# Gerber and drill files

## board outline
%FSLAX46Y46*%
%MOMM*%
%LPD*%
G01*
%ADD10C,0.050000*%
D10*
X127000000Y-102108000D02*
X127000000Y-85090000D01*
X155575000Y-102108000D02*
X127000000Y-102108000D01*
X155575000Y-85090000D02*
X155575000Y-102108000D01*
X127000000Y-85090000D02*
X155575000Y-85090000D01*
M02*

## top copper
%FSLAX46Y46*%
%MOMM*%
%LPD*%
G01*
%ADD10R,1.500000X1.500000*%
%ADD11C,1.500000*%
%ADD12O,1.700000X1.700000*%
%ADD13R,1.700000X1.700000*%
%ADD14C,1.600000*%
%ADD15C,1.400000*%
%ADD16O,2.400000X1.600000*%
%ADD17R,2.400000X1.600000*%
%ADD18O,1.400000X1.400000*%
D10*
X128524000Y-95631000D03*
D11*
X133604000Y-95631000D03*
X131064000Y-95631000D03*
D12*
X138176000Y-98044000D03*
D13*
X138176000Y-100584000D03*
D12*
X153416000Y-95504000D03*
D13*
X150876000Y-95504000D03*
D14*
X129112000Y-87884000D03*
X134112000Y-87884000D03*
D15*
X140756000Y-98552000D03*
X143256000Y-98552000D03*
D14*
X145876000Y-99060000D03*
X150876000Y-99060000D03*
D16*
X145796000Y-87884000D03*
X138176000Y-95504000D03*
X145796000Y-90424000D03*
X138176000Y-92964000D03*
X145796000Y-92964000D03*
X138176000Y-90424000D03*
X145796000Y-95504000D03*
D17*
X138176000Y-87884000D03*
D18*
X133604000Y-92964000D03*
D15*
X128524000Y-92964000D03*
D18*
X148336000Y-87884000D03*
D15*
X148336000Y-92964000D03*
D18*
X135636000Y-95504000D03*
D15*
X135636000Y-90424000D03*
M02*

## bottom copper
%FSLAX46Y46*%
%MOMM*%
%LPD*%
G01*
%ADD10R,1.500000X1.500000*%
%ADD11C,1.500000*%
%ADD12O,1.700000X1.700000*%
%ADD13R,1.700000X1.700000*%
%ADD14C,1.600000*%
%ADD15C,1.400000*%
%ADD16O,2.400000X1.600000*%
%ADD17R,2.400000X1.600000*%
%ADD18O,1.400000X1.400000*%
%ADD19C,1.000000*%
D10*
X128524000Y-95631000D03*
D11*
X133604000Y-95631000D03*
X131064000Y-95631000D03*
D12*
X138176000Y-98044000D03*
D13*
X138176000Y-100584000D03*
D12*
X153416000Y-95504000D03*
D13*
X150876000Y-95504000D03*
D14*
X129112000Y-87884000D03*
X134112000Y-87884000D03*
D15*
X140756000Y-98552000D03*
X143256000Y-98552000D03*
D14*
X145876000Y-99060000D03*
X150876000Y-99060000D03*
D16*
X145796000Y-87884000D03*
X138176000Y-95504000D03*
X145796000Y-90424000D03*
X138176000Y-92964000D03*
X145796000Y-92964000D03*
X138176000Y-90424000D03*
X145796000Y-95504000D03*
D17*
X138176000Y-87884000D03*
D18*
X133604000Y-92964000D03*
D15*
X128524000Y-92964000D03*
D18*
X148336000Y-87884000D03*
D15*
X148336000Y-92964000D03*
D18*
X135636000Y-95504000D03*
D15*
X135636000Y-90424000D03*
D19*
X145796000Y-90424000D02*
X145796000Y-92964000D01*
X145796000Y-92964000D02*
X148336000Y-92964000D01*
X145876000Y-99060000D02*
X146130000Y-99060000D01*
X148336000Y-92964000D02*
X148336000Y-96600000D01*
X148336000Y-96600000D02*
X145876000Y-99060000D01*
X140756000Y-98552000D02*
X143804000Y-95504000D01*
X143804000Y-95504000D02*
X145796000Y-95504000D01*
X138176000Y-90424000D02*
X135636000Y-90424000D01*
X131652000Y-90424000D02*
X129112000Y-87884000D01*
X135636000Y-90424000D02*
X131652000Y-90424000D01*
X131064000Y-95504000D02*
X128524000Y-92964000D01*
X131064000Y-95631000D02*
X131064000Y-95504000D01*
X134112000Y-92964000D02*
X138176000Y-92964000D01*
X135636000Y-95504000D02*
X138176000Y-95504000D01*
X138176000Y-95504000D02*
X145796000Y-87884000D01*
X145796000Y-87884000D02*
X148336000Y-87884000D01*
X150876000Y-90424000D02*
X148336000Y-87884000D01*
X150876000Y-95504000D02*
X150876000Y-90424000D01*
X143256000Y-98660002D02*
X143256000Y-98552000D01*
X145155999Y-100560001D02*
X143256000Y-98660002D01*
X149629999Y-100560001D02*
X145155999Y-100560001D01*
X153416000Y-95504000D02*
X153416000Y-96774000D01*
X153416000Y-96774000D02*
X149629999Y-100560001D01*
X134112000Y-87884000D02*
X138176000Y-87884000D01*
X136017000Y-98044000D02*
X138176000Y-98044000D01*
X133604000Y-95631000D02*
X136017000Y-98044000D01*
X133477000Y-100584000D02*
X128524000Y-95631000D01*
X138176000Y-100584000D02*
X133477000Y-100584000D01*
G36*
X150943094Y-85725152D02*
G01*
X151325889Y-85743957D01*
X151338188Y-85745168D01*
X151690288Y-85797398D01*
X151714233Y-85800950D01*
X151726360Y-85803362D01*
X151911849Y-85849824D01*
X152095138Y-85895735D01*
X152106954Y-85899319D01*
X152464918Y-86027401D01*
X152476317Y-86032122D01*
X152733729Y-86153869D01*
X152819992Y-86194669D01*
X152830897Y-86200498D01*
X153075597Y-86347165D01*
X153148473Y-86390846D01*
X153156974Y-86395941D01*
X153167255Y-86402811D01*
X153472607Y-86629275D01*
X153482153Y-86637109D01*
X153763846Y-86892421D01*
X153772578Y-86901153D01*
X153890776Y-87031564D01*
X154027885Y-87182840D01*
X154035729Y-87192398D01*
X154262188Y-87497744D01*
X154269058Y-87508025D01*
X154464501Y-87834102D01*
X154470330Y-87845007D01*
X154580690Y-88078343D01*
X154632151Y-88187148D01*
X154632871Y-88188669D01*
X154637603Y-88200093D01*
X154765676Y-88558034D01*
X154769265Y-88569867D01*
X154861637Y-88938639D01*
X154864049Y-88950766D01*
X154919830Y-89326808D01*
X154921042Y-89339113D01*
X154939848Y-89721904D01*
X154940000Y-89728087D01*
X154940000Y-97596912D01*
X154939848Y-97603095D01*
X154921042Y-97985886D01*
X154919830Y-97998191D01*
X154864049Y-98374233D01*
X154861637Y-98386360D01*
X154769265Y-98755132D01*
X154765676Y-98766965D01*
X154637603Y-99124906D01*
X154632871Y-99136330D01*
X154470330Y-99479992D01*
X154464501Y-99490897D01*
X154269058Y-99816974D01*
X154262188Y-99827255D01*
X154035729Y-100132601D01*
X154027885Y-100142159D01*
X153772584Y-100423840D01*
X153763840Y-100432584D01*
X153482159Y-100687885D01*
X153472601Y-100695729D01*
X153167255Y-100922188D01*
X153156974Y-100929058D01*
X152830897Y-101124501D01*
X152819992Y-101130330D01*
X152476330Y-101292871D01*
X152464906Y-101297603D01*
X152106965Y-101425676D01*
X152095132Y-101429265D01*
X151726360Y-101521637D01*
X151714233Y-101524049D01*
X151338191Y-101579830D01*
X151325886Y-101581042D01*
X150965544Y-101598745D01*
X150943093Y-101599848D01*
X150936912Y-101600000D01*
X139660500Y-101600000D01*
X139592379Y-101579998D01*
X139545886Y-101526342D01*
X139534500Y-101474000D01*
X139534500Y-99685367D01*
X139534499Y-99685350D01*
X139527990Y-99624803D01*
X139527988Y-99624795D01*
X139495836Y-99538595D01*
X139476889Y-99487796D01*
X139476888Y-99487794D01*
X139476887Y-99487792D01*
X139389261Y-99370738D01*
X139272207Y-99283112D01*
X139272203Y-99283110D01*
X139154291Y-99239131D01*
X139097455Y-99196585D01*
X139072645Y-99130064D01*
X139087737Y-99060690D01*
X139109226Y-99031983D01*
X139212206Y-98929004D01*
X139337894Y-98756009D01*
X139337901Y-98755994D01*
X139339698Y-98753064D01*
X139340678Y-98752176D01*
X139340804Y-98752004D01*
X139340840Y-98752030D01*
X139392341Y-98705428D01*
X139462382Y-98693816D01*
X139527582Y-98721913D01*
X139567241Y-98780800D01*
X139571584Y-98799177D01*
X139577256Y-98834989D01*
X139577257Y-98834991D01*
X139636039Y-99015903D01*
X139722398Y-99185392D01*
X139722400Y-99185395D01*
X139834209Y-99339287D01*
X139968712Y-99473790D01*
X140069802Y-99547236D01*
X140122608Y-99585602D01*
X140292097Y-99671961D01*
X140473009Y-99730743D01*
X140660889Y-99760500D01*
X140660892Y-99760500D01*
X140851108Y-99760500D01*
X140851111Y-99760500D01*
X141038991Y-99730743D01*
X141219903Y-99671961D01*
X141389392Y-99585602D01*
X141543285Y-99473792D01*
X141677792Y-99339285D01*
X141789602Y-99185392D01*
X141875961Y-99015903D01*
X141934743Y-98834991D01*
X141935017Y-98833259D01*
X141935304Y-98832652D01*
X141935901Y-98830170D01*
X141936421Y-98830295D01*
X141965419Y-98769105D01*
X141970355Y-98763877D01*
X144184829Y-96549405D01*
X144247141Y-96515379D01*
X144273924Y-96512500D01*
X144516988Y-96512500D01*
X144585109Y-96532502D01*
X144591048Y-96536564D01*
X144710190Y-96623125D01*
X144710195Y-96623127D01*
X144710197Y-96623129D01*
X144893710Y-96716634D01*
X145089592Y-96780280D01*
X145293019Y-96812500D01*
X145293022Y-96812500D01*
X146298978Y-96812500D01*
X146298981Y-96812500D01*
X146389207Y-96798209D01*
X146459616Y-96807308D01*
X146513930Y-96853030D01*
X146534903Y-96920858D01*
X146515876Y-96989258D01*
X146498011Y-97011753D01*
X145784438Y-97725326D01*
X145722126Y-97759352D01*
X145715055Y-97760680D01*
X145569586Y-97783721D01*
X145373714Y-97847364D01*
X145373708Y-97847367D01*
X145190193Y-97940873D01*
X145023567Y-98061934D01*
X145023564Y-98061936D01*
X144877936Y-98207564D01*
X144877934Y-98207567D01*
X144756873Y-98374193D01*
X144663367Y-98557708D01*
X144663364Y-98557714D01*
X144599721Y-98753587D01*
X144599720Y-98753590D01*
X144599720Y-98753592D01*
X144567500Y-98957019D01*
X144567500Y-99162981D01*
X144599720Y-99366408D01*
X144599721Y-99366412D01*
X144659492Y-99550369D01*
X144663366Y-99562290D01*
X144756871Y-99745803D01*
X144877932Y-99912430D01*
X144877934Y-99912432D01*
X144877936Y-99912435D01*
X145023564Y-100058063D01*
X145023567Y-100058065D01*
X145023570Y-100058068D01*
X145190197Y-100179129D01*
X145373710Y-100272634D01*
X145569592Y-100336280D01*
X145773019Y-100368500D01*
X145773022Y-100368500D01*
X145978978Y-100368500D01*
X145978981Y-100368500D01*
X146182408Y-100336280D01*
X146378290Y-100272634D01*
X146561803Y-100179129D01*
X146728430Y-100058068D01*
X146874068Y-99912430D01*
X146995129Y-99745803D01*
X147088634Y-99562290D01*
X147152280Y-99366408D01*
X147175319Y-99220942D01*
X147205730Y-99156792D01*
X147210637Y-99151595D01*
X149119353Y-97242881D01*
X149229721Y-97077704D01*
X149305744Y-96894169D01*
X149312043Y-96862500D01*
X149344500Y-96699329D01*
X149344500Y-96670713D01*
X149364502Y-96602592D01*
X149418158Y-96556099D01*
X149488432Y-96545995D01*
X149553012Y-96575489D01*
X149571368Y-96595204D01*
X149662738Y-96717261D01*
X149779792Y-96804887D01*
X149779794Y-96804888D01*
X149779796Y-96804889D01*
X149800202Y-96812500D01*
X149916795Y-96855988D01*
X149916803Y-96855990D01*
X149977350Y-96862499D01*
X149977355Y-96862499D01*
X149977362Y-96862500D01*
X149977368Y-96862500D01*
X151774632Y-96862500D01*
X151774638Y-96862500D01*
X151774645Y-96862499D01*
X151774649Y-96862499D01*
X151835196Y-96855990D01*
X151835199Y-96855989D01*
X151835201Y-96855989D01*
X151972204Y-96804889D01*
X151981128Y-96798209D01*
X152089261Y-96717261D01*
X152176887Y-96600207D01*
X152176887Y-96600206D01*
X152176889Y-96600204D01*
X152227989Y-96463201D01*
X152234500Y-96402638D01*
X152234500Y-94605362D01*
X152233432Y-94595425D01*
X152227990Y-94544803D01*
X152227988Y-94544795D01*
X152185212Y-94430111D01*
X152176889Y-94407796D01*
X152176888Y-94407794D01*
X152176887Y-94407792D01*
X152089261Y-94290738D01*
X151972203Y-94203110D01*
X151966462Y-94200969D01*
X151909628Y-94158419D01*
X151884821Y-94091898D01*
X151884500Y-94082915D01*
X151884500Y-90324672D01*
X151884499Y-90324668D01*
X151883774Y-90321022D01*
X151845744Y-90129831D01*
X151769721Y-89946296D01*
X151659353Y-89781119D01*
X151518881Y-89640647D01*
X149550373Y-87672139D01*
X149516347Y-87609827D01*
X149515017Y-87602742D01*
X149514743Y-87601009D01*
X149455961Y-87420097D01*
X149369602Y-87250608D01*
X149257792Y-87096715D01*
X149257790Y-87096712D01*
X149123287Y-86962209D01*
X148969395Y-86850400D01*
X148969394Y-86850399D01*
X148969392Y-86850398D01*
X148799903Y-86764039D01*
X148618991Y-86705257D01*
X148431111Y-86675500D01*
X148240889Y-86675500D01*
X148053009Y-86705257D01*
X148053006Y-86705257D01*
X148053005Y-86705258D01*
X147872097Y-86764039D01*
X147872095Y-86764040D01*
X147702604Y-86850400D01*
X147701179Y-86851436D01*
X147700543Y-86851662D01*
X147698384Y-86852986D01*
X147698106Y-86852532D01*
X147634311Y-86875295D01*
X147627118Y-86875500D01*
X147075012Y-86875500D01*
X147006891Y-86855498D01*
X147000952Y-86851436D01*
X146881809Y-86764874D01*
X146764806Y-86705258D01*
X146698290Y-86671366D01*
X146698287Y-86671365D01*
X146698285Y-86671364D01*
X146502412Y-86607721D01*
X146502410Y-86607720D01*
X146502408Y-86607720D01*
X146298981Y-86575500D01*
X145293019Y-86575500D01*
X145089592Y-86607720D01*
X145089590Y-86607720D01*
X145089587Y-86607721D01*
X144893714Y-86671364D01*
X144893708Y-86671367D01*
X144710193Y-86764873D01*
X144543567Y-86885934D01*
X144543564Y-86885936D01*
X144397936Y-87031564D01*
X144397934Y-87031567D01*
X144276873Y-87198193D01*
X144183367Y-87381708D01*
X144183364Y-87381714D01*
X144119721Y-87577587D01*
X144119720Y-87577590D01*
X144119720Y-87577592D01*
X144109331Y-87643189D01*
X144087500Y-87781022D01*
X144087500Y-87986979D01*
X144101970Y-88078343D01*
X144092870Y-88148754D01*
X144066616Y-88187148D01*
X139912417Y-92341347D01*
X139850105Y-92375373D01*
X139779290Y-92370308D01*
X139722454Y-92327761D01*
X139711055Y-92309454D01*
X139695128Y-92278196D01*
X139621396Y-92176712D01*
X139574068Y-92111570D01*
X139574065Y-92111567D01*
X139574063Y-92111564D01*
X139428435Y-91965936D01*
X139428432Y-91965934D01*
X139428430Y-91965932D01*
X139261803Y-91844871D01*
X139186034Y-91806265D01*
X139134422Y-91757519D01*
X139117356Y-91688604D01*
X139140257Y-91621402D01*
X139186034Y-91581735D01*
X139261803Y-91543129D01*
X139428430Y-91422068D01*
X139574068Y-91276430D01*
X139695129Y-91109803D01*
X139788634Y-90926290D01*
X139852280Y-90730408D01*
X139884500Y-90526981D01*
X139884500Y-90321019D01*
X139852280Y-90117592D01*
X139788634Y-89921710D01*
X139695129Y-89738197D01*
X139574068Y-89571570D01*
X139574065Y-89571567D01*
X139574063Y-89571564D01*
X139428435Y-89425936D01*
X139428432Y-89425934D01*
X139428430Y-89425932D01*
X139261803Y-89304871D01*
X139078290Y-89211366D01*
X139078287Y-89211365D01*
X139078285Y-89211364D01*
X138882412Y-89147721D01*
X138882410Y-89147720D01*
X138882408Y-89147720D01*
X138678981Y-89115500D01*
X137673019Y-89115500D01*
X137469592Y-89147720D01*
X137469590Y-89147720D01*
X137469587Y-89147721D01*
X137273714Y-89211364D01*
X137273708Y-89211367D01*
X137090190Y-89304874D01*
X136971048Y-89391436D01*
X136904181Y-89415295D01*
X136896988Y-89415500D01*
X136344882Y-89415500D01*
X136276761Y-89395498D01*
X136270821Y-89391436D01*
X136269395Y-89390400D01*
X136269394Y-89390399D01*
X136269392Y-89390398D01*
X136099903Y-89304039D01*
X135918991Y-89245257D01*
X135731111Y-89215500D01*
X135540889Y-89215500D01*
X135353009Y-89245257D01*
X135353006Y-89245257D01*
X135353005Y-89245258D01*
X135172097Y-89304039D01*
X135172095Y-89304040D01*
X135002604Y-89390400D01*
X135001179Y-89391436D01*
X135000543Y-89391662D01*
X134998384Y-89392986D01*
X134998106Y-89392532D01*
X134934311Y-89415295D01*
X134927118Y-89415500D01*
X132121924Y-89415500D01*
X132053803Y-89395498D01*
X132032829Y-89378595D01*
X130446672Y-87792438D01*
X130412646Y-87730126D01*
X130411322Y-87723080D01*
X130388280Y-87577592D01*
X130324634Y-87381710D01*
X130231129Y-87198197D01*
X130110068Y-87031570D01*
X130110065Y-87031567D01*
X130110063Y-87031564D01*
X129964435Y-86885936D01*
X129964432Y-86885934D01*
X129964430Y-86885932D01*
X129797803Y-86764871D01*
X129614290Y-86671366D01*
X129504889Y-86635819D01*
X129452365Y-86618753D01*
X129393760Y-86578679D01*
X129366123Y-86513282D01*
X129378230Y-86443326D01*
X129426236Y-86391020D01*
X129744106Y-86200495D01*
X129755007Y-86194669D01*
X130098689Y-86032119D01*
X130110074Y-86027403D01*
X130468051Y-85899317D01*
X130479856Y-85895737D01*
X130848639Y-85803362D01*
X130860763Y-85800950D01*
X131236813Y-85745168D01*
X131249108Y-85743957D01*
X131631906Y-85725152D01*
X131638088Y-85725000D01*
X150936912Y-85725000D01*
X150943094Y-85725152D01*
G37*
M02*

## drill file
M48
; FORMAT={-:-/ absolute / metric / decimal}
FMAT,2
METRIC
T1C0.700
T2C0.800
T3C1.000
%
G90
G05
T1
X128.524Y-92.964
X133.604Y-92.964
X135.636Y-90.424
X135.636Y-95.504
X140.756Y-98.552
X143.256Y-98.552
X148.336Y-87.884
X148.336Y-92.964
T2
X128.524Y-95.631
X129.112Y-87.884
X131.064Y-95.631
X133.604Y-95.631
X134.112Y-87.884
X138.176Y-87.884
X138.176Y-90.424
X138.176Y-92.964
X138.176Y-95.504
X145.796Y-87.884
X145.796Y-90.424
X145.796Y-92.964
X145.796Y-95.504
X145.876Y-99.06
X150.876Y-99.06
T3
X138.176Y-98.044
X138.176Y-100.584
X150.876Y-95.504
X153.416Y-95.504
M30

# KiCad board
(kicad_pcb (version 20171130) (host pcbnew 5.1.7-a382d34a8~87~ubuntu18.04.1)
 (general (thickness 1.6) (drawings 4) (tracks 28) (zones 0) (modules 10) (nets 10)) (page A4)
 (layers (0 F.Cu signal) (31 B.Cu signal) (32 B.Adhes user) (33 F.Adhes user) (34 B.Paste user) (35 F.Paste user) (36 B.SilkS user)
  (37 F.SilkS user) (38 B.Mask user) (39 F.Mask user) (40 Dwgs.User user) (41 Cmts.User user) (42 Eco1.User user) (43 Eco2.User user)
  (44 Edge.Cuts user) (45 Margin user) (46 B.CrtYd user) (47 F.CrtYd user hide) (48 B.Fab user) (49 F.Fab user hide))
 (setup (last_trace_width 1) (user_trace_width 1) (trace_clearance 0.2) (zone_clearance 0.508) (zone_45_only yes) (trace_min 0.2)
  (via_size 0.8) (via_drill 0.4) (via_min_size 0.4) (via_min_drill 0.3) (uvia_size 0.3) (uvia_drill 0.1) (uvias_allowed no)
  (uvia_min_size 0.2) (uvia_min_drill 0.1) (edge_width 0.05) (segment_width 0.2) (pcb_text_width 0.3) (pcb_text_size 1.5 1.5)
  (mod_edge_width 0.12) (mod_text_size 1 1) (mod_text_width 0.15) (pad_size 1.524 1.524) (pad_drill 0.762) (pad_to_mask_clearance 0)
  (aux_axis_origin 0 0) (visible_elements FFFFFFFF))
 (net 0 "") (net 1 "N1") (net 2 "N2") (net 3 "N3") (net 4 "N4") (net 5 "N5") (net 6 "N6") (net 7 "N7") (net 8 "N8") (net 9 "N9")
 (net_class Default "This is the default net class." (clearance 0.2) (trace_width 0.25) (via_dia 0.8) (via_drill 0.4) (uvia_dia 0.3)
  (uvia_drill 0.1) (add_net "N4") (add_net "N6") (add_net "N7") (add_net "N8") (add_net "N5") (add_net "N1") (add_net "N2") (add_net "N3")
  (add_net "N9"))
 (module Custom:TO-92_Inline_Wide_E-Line (layer F.Cu) (at 128.524 95.631)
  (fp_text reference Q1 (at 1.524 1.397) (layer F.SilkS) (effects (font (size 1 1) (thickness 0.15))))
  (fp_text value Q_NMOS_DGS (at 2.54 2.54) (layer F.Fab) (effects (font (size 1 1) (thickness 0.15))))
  (pad 1 thru_hole rect (at 0 0 90) (size 1.5 1.5) (drill 0.8) (layers *.Cu *.Mask) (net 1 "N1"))
  (pad 3 thru_hole circle (at 5.08 0 90) (size 1.5 1.5) (drill 0.8) (layers *.Cu *.Mask) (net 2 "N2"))
  (pad 2 thru_hole circle (at 2.54 0 90) (size 1.5 1.5) (drill 0.8) (layers *.Cu *.Mask) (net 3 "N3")))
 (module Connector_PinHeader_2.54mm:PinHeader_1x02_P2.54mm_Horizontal (layer F.Cu) (at 138.176 100.584 180)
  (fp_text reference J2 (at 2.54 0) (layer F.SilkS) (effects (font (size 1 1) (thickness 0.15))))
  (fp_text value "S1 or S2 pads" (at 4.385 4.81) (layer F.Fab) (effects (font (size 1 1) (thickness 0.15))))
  (pad 2 thru_hole oval (at 0 2.54 180) (size 1.7 1.7) (drill 1) (layers *.Cu *.Mask) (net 2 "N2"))
  (pad 1 thru_hole rect (at 0 0 180) (size 1.7 1.7) (drill 1) (layers *.Cu *.Mask) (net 1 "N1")))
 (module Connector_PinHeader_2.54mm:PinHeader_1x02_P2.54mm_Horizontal (layer F.Cu) (at 150.876 95.504 90)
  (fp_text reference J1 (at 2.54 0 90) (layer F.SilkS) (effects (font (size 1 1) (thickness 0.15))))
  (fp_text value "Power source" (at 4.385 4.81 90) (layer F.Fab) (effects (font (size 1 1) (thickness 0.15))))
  (pad 2 thru_hole oval (at 0 2.54 90) (size 1.7 1.7) (drill 1) (layers *.Cu *.Mask) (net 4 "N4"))
  (pad 1 thru_hole rect (at 0 0 90) (size 1.7 1.7) (drill 1) (layers *.Cu *.Mask) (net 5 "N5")))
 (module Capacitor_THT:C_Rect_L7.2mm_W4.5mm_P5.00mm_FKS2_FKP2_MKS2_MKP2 (layer F.Cu) (at 134.112 87.884 180)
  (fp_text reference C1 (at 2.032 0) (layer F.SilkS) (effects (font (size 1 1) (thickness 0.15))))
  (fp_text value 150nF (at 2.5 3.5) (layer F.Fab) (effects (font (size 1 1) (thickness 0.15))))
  (pad 2 thru_hole circle (at 5 0 180) (size 1.6 1.6) (drill 0.8) (layers *.Cu *.Mask) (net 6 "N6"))
  (pad 1 thru_hole circle (at 0 0 180) (size 1.6 1.6) (drill 0.8) (layers *.Cu *.Mask) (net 4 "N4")))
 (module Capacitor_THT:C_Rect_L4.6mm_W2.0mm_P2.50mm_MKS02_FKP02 (layer F.Cu) (at 143.256 98.552 180)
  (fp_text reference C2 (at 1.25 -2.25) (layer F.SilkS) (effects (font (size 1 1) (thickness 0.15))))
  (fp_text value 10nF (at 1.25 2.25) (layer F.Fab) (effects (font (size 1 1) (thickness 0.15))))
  (pad 2 thru_hole circle (at 2.5 0 180) (size 1.4 1.4) (drill 0.7) (layers *.Cu *.Mask) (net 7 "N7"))
  (pad 1 thru_hole circle (at 0 0 180) (size 1.4 1.4) (drill 0.7) (layers *.Cu *.Mask) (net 4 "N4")))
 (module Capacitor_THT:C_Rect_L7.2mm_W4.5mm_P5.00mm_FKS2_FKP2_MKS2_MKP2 (layer F.Cu) (at 150.876 99.06 180)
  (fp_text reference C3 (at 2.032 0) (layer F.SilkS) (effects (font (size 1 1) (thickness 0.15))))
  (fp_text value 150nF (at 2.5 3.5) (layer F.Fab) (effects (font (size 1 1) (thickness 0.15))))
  (pad 2 thru_hole circle (at 5 0 180) (size 1.6 1.6) (drill 0.8) (layers *.Cu *.Mask) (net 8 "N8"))
  (pad 1 thru_hole circle (at 0 0 180) (size 1.6 1.6) (drill 0.8) (layers *.Cu *.Mask) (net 4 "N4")))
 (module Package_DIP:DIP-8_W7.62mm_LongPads (layer F.Cu) (at 138.176 87.884)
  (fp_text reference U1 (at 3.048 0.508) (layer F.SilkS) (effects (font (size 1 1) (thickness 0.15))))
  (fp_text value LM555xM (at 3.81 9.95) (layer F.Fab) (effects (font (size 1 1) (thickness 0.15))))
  (pad 8 thru_hole oval (at 7.62 0) (size 2.4 1.6) (drill 0.8) (layers *.Cu *.Mask) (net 5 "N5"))
  (pad 4 thru_hole oval (at 0 7.62) (size 2.4 1.6) (drill 0.8) (layers *.Cu *.Mask) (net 5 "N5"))
  (pad 7 thru_hole oval (at 7.62 2.54) (size 2.4 1.6) (drill 0.8) (layers *.Cu *.Mask) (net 8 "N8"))
  (pad 3 thru_hole oval (at 0 5.08) (size 2.4 1.6) (drill 0.8) (layers *.Cu *.Mask) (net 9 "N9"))
  (pad 6 thru_hole oval (at 7.62 5.08) (size 2.4 1.6) (drill 0.8) (layers *.Cu *.Mask) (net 8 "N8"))
  (pad 2 thru_hole oval (at 0 2.54) (size 2.4 1.6) (drill 0.8) (layers *.Cu *.Mask) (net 6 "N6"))
  (pad 5 thru_hole oval (at 7.62 7.62) (size 2.4 1.6) (drill 0.8) (layers *.Cu *.Mask) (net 7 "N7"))
  (pad 1 thru_hole rect (at 0 0) (size 2.4 1.6) (drill 0.8) (layers *.Cu *.Mask) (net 4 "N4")))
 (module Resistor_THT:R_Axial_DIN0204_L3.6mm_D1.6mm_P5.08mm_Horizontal (layer F.Cu) (at 128.524 92.964)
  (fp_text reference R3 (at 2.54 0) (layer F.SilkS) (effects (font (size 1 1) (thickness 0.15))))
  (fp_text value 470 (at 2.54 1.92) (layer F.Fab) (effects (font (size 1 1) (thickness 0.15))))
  (pad 2 thru_hole oval (at 5.08 0) (size 1.4 1.4) (drill 0.7) (layers *.Cu *.Mask) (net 9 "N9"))
  (pad 1 thru_hole circle (at 0 0) (size 1.4 1.4) (drill 0.7) (layers *.Cu *.Mask) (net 3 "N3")))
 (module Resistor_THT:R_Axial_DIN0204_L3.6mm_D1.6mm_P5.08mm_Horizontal (layer F.Cu) (at 148.336 92.964 90)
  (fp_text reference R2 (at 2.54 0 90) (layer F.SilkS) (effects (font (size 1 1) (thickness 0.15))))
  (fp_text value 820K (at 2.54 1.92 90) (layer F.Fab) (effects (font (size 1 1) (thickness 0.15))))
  (pad 2 thru_hole oval (at 5.08 0 90) (size 1.4 1.4) (drill 0.7) (layers *.Cu *.Mask) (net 5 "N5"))
  (pad 1 thru_hole circle (at 0 0 90) (size 1.4 1.4) (drill 0.7) (layers *.Cu *.Mask) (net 8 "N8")))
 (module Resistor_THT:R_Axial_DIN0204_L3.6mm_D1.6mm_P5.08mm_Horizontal (layer F.Cu) (at 135.636 90.424 270)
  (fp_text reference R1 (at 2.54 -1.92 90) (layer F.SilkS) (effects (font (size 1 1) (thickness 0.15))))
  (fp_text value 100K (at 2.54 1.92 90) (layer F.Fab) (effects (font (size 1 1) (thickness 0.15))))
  (pad 2 thru_hole oval (at 5.08 0 270) (size 1.4 1.4) (drill 0.7) (layers *.Cu *.Mask) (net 5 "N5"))
  (pad 1 thru_hole circle (at 0 0 270) (size 1.4 1.4) (drill 0.7) (layers *.Cu *.Mask) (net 6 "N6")))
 (gr_line (start 127 102.108) (end 127 85.09) (layer Edge.Cuts) (width 0.05))
 (gr_line (start 155.575 102.108) (end 127 102.108) (layer Edge.Cuts) (width 0.05))
 (gr_line (start 155.575 85.09) (end 155.575 102.108) (layer Edge.Cuts) (width 0.05))
 (gr_line (start 127 85.09) (end 155.575 85.09) (layer Edge.Cuts) (width 0.05))
 (segment (start 145.796 90.424) (end 145.796 92.964) (width 1) (layer B.Cu) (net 8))
 (segment (start 145.796 92.964) (end 148.336 92.964) (width 1) (layer B.Cu) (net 8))
 (segment (start 145.876 99.06) (end 146.13 99.06) (width 1) (layer B.Cu) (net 8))
 (segment (start 148.336 92.964) (end 148.336 96.6) (width 1) (layer B.Cu) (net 8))
 (segment (start 148.336 96.6) (end 145.876 99.06) (width 1) (layer B.Cu) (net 8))
 (segment (start 140.756 98.552) (end 143.804 95.504) (width 1) (layer B.Cu) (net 7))
 (segment (start 143.804 95.504) (end 145.796 95.504) (width 1) (layer B.Cu) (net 7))
 (segment (start 138.176 90.424) (end 135.636 90.424) (width 1) (layer B.Cu) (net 6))
 (segment (start 131.652 90.424) (end 129.112 87.884) (width 1) (layer B.Cu) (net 6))
 (segment (start 135.636 90.424) (end 131.652 90.424) (width 1) (layer B.Cu) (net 6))
 (segment (start 131.064 95.504) (end 128.524 92.964) (width 1) (layer B.Cu) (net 3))
 (segment (start 131.064 95.631) (end 131.064 95.504) (width 1) (layer B.Cu) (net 3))
 (segment (start 134.112 92.964) (end 138.176 92.964) (width 1) (layer B.Cu) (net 9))
 (segment (start 135.636 95.504) (end 138.176 95.504) (width 1) (layer B.Cu) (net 5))
 (segment (start 138.176 95.504) (end 145.796 87.884) (width 1) (layer B.Cu) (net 5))
 (segment (start 145.796 87.884) (end 148.336 87.884) (width 1) (layer B.Cu) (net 5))
 (segment (start 150.876 90.424) (end 148.336 87.884) (width 1) (layer B.Cu) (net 5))
 (segment (start 150.876 95.504) (end 150.876 90.424) (width 1) (layer B.Cu) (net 5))
 (segment (start 143.256 98.660002) (end 143.256 98.552) (width 1) (layer B.Cu) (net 4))
 (segment (start 145.155999 100.560001) (end 143.256 98.660002) (width 1) (layer B.Cu) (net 4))
 (segment (start 149.629999 100.560001) (end 145.155999 100.560001) (width 1) (layer B.Cu) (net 4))
 (segment (start 153.416 95.504) (end 153.416 96.774) (width 1) (layer B.Cu) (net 4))
 (segment (start 153.416 96.774) (end 149.629999 100.560001) (width 1) (layer B.Cu) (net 4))
 (segment (start 134.112 87.884) (end 138.176 87.884) (width 1) (layer B.Cu) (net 4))
 (segment (start 136.017 98.044) (end 138.176 98.044) (width 1) (layer B.Cu) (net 2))
 (segment (start 133.604 95.631) (end 136.017 98.044) (width 1) (layer B.Cu) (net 2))
 (segment (start 133.477 100.584) (end 128.524 95.631) (width 1) (layer B.Cu) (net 1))
 (segment (start 138.176 100.584) (end 133.477 100.584) (width 1) (layer B.Cu) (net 1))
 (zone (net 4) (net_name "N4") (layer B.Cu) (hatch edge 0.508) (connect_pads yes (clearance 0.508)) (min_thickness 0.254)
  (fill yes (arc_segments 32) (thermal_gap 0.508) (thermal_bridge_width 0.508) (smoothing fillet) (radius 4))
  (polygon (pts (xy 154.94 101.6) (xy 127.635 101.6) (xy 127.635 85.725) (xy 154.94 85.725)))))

